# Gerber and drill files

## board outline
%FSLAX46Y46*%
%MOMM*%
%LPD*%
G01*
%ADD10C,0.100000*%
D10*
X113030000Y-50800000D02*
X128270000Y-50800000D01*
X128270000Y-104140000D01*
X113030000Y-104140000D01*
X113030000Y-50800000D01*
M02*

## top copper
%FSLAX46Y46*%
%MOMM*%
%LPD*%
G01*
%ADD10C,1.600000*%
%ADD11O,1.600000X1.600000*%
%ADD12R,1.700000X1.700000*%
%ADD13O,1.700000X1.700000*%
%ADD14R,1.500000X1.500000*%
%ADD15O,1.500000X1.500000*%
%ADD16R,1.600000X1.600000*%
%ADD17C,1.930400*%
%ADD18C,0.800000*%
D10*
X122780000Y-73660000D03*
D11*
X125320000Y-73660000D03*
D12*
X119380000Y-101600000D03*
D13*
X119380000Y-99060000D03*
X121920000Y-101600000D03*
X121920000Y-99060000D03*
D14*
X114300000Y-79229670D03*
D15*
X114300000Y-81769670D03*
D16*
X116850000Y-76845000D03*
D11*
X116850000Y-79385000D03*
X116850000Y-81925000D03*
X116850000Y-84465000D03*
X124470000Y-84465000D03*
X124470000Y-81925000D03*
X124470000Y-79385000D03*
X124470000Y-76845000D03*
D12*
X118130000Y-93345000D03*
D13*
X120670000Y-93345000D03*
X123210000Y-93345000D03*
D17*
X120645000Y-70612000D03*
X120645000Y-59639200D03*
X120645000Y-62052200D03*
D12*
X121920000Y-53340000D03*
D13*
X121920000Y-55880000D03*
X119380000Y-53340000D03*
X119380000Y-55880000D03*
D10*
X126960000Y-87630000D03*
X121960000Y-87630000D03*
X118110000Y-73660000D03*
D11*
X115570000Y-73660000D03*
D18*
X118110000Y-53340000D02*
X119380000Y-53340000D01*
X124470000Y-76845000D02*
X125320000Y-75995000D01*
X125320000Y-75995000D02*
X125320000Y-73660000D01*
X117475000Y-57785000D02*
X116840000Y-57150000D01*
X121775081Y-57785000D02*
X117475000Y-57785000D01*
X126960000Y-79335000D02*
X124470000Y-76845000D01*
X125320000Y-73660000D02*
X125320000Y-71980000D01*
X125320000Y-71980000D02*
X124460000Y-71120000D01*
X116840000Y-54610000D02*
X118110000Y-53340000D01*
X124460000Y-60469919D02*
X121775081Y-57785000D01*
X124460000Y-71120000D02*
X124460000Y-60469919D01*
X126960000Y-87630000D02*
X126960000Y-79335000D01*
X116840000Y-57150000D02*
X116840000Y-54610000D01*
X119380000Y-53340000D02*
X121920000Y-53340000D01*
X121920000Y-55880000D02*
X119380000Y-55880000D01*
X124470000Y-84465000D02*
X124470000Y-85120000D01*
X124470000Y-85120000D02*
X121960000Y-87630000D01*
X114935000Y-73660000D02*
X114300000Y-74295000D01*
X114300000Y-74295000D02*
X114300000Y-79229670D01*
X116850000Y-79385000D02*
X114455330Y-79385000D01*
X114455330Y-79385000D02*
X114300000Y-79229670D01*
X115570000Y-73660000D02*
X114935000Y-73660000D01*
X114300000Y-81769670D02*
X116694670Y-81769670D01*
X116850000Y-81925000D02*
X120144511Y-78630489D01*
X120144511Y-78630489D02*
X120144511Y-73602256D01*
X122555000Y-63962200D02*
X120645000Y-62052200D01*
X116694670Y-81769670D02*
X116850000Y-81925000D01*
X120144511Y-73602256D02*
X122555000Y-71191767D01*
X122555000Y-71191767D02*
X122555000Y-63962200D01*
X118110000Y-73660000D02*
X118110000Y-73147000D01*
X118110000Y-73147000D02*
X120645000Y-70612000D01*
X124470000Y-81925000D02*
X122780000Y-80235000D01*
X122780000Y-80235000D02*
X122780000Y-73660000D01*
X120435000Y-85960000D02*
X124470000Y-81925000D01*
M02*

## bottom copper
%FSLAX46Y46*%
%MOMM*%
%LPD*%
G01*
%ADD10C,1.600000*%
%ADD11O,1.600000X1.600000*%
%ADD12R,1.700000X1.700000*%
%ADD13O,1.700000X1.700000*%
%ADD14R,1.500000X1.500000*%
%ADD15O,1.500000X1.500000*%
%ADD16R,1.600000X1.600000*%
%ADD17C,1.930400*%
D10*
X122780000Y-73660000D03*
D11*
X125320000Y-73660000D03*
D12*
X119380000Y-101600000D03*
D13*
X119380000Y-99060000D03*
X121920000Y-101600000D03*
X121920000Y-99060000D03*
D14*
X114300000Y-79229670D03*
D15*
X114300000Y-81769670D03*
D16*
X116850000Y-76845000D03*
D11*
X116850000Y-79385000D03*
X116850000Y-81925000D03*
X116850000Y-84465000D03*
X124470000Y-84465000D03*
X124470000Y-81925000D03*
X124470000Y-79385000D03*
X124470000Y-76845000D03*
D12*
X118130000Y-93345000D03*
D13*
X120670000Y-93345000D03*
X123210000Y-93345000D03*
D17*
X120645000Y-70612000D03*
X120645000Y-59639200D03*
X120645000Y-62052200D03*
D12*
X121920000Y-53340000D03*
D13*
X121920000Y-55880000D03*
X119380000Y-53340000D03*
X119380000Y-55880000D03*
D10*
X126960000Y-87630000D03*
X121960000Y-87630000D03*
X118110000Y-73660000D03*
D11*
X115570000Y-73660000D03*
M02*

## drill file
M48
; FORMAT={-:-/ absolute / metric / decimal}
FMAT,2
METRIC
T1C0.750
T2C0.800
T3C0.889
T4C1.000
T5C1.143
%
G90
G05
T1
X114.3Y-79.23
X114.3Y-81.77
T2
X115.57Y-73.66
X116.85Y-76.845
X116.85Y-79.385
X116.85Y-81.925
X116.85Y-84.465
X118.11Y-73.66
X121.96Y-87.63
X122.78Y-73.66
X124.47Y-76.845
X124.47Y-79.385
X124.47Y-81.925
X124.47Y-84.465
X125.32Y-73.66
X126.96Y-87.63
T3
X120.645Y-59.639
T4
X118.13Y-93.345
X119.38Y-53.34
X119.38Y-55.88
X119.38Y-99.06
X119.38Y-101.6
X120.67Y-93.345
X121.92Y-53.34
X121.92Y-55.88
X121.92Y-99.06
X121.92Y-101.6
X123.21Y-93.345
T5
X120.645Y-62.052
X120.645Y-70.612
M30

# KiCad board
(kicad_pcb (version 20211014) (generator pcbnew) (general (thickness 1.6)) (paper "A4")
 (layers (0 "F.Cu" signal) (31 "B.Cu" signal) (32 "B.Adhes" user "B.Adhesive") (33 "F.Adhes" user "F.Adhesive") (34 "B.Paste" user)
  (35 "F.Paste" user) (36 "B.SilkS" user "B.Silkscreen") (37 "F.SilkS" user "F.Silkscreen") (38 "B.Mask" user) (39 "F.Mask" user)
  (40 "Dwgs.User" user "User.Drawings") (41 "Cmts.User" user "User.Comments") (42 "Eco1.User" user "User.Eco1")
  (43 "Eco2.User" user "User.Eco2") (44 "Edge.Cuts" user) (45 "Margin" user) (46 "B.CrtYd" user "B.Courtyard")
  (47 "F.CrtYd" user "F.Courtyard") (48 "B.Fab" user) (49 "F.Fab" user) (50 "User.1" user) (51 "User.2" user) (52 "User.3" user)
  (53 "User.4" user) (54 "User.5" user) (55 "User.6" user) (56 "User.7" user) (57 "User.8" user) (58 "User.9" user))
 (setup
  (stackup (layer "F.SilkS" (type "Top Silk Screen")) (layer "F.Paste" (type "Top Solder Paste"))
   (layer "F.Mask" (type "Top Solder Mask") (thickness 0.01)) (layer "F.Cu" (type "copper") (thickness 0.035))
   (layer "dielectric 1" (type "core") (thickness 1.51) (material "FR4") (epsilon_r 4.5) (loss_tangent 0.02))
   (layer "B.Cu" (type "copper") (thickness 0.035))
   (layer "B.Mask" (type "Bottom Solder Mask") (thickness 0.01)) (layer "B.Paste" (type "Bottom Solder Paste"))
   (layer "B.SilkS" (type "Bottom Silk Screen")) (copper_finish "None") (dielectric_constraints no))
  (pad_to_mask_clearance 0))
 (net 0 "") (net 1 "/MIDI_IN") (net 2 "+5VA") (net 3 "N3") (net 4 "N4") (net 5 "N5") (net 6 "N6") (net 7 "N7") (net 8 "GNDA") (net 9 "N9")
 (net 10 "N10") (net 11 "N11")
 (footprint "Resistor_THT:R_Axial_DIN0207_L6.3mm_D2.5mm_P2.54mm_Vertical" (layer "F.Cu") (at 122.78 73.66)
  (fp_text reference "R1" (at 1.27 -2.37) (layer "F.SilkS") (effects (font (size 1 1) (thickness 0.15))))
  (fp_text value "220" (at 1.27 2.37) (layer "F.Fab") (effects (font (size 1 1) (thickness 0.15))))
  (pad "1" thru_hole circle (at 0 0) (size 1.6 1.6) (drill 0.8) (layers *.Cu *.Mask) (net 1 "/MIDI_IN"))
  (pad "2" thru_hole oval (at 2.54 0) (size 1.6 1.6) (drill 0.8) (layers *.Cu *.Mask) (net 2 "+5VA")))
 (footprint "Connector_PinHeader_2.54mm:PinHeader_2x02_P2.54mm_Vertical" (layer "F.Cu") (at 119.38 101.6 90)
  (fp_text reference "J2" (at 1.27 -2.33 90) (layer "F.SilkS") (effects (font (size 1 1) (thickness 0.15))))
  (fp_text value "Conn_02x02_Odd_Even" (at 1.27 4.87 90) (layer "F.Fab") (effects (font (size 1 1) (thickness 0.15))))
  (pad "1" thru_hole rect (at 0 0 90) (size 1.7 1.7) (drill 1) (layers *.Cu *.Mask) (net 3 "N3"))
  (pad "2" thru_hole oval (at 2.54 0 90) (size 1.7 1.7) (drill 1) (layers *.Cu *.Mask) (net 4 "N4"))
  (pad "3" thru_hole oval (at 0 2.54 90) (size 1.7 1.7) (drill 1) (layers *.Cu *.Mask) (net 3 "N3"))
  (pad "4" thru_hole oval (at 2.54 2.54 90) (size 1.7 1.7) (drill 1) (layers *.Cu *.Mask) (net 4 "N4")))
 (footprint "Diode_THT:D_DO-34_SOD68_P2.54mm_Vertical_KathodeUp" (layer "F.Cu") (at 114.3 79.22967 -90)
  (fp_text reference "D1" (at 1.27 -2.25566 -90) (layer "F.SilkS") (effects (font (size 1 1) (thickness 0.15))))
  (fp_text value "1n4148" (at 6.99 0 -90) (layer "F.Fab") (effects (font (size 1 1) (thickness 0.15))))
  (pad "1" thru_hole rect (at 0 0 270) (size 1.5 1.5) (drill 0.75) (layers *.Cu *.Mask) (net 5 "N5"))
  (pad "2" thru_hole oval (at 2.54 0 270) (size 1.5 1.5) (drill 0.75) (layers *.Cu *.Mask) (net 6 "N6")))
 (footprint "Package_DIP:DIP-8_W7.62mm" (layer "F.Cu") (at 116.85 76.845)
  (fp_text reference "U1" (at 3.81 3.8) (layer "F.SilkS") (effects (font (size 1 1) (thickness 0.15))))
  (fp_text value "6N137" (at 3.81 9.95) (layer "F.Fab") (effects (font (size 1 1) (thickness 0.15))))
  (pad "1" thru_hole rect (at 0 0) (size 1.6 1.6) (drill 0.8) (layers *.Cu *.Mask) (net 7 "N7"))
  (pad "2" thru_hole oval (at 0 2.54) (size 1.6 1.6) (drill 0.8) (layers *.Cu *.Mask) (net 5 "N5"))
  (pad "3" thru_hole oval (at 0 5.08) (size 1.6 1.6) (drill 0.8) (layers *.Cu *.Mask) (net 6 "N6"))
  (pad "4" thru_hole oval (at 0 7.62) (size 1.6 1.6) (drill 0.8) (layers *.Cu *.Mask))
  (pad "5" thru_hole oval (at 7.62 7.62) (size 1.6 1.6) (drill 0.8) (layers *.Cu *.Mask) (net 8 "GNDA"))
  (pad "6" thru_hole oval (at 7.62 5.08) (size 1.6 1.6) (drill 0.8) (layers *.Cu *.Mask) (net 1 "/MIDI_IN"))
  (pad "7" thru_hole oval (at 7.62 2.54) (size 1.6 1.6) (drill 0.8) (layers *.Cu *.Mask) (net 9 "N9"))
  (pad "8" thru_hole oval (at 7.62 0) (size 1.6 1.6) (drill 0.8) (layers *.Cu *.Mask) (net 2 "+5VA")))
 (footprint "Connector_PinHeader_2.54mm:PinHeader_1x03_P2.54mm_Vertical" (layer "F.Cu") (at 118.13 93.345 90)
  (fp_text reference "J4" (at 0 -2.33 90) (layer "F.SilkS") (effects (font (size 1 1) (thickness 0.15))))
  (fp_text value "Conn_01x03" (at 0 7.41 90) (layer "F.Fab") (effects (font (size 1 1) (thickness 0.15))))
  (pad "1" thru_hole rect (at 0 0 90) (size 1.7 1.7) (drill 1) (layers *.Cu *.Mask) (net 2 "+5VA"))
  (pad "2" thru_hole oval (at 0 2.54 90) (size 1.7 1.7) (drill 1) (layers *.Cu *.Mask) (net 1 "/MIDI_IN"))
  (pad "3" thru_hole oval (at 0 5.08 90) (size 1.7 1.7) (drill 1) (layers *.Cu *.Mask) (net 8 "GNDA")))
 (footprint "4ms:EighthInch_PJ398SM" (layer "F.Cu") (at 120.645 65.405 90)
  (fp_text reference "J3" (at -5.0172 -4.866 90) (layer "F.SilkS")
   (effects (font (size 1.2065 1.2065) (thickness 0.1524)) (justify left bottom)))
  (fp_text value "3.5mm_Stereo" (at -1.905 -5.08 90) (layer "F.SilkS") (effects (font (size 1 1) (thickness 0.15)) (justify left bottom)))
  (pad "1" thru_hole circle locked (at -5.207 0 90) (size 1.9304 1.9304) (drill 1.143) (layers *.Cu *.Mask) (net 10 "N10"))
  (pad "2" thru_hole circle locked (at 5.7658 0 90) (size 1.9304 1.9304) (drill 0.889) (layers *.Cu *.Mask) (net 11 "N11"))
  (pad "3" thru_hole circle locked (at 3.3528 0 90) (size 1.9304 1.9304) (drill 1.143) (layers *.Cu *.Mask) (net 6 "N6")))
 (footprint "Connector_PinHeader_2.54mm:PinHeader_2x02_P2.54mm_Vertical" (layer "F.Cu") (at 121.92 53.34 -90)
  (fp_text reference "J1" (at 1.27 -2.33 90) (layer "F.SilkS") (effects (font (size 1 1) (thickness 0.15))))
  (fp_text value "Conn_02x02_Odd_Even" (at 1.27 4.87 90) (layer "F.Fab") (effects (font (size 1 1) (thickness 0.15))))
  (pad "1" thru_hole rect (at 0 0 270) (size 1.7 1.7) (drill 1) (layers *.Cu *.Mask) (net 2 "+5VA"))
  (pad "2" thru_hole oval (at 2.54 0 270) (size 1.7 1.7) (drill 1) (layers *.Cu *.Mask) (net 8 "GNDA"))
  (pad "3" thru_hole oval (at 0 2.54 270) (size 1.7 1.7) (drill 1) (layers *.Cu *.Mask) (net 2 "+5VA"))
  (pad "4" thru_hole oval (at 2.54 2.54 270) (size 1.7 1.7) (drill 1) (layers *.Cu *.Mask) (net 8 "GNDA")))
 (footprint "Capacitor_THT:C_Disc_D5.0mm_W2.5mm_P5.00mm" (layer "F.Cu") (at 126.96 87.63 180)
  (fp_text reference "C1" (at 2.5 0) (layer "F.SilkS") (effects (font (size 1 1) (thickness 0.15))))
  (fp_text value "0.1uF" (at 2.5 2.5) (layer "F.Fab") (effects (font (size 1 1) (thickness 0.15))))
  (pad "1" thru_hole circle (at 0 0 180) (size 1.6 1.6) (drill 0.8) (layers *.Cu *.Mask) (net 2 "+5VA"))
  (pad "2" thru_hole circle (at 5 0 180) (size 1.6 1.6) (drill 0.8) (layers *.Cu *.Mask) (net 8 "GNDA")))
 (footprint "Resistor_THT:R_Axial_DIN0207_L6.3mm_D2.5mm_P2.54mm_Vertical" (layer "F.Cu") (at 118.11 73.66 180)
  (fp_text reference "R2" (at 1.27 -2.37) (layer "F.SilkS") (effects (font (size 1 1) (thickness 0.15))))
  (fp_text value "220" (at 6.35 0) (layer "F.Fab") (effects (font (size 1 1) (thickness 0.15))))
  (pad "1" thru_hole circle (at 0 0 180) (size 1.6 1.6) (drill 0.8) (layers *.Cu *.Mask) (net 10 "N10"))
  (pad "2" thru_hole oval (at 2.54 0 180) (size 1.6 1.6) (drill 0.8) (layers *.Cu *.Mask) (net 5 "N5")))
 (gr_rect (start 113.03 50.8) (end 128.27 104.14) (layer "Edge.Cuts") (width 0.1) (fill none))
 (segment (start 118.11 53.34) (end 119.38 53.34) (width 0.8) (layer "F.Cu") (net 2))
 (segment (start 124.47 76.845) (end 125.32 75.995) (width 0.8) (layer "F.Cu") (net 2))
 (segment (start 125.32 75.995) (end 125.32 73.66) (width 0.8) (layer "F.Cu") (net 2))
 (segment (start 117.475 57.785) (end 116.84 57.15) (width 0.8) (layer "F.Cu") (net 2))
 (segment (start 121.775081 57.785) (end 117.475 57.785) (width 0.8) (layer "F.Cu") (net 2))
 (segment (start 126.96 79.335) (end 124.47 76.845) (width 0.8) (layer "F.Cu") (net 2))
 (segment (start 125.32 73.66) (end 125.32 71.98) (width 0.8) (layer "F.Cu") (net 2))
 (segment (start 125.32 71.98) (end 124.46 71.12) (width 0.8) (layer "F.Cu") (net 2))
 (segment (start 116.84 54.61) (end 118.11 53.34) (width 0.8) (layer "F.Cu") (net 2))
 (segment (start 124.46 60.469919) (end 121.775081 57.785) (width 0.8) (layer "F.Cu") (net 2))
 (segment (start 124.46 71.12) (end 124.46 60.469919) (width 0.8) (layer "F.Cu") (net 2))
 (segment (start 126.96 87.63) (end 126.96 79.335) (width 0.8) (layer "F.Cu") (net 2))
 (segment (start 116.84 57.15) (end 116.84 54.61) (width 0.8) (layer "F.Cu") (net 2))
 (segment (start 119.38 53.34) (end 121.92 53.34) (width 0.8) (layer "F.Cu") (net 2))
 (segment (start 121.92 55.88) (end 119.38 55.88) (width 0.8) (layer "F.Cu") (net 8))
 (segment (start 124.47 84.465) (end 124.47 85.12) (width 0.8) (layer "F.Cu") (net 8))
 (segment (start 124.47 85.12) (end 121.96 87.63) (width 0.8) (layer "F.Cu") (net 8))
 (segment (start 114.935 73.66) (end 114.3 74.295) (width 0.8) (layer "F.Cu") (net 5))
 (segment (start 114.3 74.295) (end 114.3 79.22967) (width 0.8) (layer "F.Cu") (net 5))
 (segment (start 116.85 79.385) (end 114.45533 79.385) (width 0.8) (layer "F.Cu") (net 5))
 (segment (start 114.45533 79.385) (end 114.3 79.22967) (width 0.8) (layer "F.Cu") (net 5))
 (segment (start 115.57 73.66) (end 114.935 73.66) (width 0.8) (layer "F.Cu") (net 5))
 (segment (start 114.3 81.76967) (end 116.69467 81.76967) (width 0.8) (layer "F.Cu") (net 6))
 (segment (start 116.85 81.925) (end 120.144511 78.630489) (width 0.8) (layer "F.Cu") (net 6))
 (segment (start 120.144511 78.630489) (end 120.144511 73.602256) (width 0.8) (layer "F.Cu") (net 6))
 (segment (start 122.555 63.9622) (end 120.645 62.0522) (width 0.8) (layer "F.Cu") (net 6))
 (segment (start 116.69467 81.76967) (end 116.85 81.925) (width 0.8) (layer "F.Cu") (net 6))
 (segment (start 120.144511 73.602256) (end 122.555 71.191767) (width 0.8) (layer "F.Cu") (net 6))
 (segment (start 122.555 71.191767) (end 122.555 63.9622) (width 0.8) (layer "F.Cu") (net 6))
 (segment (start 118.11 73.66) (end 118.11 73.147) (width 0.8) (layer "F.Cu") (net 10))
 (segment (start 118.11 73.147) (end 120.645 70.612) (width 0.8) (layer "F.Cu") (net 10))
 (segment (start 124.47 81.925) (end 122.78 80.235) (width 0.8) (layer "F.Cu") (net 1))
 (segment (start 122.78 80.235) (end 122.78 73.66) (width 0.8) (layer "F.Cu") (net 1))
 (segment (start 120.435 85.96) (end 124.47 81.925) (width 0.8) (layer "F.Cu") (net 1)))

